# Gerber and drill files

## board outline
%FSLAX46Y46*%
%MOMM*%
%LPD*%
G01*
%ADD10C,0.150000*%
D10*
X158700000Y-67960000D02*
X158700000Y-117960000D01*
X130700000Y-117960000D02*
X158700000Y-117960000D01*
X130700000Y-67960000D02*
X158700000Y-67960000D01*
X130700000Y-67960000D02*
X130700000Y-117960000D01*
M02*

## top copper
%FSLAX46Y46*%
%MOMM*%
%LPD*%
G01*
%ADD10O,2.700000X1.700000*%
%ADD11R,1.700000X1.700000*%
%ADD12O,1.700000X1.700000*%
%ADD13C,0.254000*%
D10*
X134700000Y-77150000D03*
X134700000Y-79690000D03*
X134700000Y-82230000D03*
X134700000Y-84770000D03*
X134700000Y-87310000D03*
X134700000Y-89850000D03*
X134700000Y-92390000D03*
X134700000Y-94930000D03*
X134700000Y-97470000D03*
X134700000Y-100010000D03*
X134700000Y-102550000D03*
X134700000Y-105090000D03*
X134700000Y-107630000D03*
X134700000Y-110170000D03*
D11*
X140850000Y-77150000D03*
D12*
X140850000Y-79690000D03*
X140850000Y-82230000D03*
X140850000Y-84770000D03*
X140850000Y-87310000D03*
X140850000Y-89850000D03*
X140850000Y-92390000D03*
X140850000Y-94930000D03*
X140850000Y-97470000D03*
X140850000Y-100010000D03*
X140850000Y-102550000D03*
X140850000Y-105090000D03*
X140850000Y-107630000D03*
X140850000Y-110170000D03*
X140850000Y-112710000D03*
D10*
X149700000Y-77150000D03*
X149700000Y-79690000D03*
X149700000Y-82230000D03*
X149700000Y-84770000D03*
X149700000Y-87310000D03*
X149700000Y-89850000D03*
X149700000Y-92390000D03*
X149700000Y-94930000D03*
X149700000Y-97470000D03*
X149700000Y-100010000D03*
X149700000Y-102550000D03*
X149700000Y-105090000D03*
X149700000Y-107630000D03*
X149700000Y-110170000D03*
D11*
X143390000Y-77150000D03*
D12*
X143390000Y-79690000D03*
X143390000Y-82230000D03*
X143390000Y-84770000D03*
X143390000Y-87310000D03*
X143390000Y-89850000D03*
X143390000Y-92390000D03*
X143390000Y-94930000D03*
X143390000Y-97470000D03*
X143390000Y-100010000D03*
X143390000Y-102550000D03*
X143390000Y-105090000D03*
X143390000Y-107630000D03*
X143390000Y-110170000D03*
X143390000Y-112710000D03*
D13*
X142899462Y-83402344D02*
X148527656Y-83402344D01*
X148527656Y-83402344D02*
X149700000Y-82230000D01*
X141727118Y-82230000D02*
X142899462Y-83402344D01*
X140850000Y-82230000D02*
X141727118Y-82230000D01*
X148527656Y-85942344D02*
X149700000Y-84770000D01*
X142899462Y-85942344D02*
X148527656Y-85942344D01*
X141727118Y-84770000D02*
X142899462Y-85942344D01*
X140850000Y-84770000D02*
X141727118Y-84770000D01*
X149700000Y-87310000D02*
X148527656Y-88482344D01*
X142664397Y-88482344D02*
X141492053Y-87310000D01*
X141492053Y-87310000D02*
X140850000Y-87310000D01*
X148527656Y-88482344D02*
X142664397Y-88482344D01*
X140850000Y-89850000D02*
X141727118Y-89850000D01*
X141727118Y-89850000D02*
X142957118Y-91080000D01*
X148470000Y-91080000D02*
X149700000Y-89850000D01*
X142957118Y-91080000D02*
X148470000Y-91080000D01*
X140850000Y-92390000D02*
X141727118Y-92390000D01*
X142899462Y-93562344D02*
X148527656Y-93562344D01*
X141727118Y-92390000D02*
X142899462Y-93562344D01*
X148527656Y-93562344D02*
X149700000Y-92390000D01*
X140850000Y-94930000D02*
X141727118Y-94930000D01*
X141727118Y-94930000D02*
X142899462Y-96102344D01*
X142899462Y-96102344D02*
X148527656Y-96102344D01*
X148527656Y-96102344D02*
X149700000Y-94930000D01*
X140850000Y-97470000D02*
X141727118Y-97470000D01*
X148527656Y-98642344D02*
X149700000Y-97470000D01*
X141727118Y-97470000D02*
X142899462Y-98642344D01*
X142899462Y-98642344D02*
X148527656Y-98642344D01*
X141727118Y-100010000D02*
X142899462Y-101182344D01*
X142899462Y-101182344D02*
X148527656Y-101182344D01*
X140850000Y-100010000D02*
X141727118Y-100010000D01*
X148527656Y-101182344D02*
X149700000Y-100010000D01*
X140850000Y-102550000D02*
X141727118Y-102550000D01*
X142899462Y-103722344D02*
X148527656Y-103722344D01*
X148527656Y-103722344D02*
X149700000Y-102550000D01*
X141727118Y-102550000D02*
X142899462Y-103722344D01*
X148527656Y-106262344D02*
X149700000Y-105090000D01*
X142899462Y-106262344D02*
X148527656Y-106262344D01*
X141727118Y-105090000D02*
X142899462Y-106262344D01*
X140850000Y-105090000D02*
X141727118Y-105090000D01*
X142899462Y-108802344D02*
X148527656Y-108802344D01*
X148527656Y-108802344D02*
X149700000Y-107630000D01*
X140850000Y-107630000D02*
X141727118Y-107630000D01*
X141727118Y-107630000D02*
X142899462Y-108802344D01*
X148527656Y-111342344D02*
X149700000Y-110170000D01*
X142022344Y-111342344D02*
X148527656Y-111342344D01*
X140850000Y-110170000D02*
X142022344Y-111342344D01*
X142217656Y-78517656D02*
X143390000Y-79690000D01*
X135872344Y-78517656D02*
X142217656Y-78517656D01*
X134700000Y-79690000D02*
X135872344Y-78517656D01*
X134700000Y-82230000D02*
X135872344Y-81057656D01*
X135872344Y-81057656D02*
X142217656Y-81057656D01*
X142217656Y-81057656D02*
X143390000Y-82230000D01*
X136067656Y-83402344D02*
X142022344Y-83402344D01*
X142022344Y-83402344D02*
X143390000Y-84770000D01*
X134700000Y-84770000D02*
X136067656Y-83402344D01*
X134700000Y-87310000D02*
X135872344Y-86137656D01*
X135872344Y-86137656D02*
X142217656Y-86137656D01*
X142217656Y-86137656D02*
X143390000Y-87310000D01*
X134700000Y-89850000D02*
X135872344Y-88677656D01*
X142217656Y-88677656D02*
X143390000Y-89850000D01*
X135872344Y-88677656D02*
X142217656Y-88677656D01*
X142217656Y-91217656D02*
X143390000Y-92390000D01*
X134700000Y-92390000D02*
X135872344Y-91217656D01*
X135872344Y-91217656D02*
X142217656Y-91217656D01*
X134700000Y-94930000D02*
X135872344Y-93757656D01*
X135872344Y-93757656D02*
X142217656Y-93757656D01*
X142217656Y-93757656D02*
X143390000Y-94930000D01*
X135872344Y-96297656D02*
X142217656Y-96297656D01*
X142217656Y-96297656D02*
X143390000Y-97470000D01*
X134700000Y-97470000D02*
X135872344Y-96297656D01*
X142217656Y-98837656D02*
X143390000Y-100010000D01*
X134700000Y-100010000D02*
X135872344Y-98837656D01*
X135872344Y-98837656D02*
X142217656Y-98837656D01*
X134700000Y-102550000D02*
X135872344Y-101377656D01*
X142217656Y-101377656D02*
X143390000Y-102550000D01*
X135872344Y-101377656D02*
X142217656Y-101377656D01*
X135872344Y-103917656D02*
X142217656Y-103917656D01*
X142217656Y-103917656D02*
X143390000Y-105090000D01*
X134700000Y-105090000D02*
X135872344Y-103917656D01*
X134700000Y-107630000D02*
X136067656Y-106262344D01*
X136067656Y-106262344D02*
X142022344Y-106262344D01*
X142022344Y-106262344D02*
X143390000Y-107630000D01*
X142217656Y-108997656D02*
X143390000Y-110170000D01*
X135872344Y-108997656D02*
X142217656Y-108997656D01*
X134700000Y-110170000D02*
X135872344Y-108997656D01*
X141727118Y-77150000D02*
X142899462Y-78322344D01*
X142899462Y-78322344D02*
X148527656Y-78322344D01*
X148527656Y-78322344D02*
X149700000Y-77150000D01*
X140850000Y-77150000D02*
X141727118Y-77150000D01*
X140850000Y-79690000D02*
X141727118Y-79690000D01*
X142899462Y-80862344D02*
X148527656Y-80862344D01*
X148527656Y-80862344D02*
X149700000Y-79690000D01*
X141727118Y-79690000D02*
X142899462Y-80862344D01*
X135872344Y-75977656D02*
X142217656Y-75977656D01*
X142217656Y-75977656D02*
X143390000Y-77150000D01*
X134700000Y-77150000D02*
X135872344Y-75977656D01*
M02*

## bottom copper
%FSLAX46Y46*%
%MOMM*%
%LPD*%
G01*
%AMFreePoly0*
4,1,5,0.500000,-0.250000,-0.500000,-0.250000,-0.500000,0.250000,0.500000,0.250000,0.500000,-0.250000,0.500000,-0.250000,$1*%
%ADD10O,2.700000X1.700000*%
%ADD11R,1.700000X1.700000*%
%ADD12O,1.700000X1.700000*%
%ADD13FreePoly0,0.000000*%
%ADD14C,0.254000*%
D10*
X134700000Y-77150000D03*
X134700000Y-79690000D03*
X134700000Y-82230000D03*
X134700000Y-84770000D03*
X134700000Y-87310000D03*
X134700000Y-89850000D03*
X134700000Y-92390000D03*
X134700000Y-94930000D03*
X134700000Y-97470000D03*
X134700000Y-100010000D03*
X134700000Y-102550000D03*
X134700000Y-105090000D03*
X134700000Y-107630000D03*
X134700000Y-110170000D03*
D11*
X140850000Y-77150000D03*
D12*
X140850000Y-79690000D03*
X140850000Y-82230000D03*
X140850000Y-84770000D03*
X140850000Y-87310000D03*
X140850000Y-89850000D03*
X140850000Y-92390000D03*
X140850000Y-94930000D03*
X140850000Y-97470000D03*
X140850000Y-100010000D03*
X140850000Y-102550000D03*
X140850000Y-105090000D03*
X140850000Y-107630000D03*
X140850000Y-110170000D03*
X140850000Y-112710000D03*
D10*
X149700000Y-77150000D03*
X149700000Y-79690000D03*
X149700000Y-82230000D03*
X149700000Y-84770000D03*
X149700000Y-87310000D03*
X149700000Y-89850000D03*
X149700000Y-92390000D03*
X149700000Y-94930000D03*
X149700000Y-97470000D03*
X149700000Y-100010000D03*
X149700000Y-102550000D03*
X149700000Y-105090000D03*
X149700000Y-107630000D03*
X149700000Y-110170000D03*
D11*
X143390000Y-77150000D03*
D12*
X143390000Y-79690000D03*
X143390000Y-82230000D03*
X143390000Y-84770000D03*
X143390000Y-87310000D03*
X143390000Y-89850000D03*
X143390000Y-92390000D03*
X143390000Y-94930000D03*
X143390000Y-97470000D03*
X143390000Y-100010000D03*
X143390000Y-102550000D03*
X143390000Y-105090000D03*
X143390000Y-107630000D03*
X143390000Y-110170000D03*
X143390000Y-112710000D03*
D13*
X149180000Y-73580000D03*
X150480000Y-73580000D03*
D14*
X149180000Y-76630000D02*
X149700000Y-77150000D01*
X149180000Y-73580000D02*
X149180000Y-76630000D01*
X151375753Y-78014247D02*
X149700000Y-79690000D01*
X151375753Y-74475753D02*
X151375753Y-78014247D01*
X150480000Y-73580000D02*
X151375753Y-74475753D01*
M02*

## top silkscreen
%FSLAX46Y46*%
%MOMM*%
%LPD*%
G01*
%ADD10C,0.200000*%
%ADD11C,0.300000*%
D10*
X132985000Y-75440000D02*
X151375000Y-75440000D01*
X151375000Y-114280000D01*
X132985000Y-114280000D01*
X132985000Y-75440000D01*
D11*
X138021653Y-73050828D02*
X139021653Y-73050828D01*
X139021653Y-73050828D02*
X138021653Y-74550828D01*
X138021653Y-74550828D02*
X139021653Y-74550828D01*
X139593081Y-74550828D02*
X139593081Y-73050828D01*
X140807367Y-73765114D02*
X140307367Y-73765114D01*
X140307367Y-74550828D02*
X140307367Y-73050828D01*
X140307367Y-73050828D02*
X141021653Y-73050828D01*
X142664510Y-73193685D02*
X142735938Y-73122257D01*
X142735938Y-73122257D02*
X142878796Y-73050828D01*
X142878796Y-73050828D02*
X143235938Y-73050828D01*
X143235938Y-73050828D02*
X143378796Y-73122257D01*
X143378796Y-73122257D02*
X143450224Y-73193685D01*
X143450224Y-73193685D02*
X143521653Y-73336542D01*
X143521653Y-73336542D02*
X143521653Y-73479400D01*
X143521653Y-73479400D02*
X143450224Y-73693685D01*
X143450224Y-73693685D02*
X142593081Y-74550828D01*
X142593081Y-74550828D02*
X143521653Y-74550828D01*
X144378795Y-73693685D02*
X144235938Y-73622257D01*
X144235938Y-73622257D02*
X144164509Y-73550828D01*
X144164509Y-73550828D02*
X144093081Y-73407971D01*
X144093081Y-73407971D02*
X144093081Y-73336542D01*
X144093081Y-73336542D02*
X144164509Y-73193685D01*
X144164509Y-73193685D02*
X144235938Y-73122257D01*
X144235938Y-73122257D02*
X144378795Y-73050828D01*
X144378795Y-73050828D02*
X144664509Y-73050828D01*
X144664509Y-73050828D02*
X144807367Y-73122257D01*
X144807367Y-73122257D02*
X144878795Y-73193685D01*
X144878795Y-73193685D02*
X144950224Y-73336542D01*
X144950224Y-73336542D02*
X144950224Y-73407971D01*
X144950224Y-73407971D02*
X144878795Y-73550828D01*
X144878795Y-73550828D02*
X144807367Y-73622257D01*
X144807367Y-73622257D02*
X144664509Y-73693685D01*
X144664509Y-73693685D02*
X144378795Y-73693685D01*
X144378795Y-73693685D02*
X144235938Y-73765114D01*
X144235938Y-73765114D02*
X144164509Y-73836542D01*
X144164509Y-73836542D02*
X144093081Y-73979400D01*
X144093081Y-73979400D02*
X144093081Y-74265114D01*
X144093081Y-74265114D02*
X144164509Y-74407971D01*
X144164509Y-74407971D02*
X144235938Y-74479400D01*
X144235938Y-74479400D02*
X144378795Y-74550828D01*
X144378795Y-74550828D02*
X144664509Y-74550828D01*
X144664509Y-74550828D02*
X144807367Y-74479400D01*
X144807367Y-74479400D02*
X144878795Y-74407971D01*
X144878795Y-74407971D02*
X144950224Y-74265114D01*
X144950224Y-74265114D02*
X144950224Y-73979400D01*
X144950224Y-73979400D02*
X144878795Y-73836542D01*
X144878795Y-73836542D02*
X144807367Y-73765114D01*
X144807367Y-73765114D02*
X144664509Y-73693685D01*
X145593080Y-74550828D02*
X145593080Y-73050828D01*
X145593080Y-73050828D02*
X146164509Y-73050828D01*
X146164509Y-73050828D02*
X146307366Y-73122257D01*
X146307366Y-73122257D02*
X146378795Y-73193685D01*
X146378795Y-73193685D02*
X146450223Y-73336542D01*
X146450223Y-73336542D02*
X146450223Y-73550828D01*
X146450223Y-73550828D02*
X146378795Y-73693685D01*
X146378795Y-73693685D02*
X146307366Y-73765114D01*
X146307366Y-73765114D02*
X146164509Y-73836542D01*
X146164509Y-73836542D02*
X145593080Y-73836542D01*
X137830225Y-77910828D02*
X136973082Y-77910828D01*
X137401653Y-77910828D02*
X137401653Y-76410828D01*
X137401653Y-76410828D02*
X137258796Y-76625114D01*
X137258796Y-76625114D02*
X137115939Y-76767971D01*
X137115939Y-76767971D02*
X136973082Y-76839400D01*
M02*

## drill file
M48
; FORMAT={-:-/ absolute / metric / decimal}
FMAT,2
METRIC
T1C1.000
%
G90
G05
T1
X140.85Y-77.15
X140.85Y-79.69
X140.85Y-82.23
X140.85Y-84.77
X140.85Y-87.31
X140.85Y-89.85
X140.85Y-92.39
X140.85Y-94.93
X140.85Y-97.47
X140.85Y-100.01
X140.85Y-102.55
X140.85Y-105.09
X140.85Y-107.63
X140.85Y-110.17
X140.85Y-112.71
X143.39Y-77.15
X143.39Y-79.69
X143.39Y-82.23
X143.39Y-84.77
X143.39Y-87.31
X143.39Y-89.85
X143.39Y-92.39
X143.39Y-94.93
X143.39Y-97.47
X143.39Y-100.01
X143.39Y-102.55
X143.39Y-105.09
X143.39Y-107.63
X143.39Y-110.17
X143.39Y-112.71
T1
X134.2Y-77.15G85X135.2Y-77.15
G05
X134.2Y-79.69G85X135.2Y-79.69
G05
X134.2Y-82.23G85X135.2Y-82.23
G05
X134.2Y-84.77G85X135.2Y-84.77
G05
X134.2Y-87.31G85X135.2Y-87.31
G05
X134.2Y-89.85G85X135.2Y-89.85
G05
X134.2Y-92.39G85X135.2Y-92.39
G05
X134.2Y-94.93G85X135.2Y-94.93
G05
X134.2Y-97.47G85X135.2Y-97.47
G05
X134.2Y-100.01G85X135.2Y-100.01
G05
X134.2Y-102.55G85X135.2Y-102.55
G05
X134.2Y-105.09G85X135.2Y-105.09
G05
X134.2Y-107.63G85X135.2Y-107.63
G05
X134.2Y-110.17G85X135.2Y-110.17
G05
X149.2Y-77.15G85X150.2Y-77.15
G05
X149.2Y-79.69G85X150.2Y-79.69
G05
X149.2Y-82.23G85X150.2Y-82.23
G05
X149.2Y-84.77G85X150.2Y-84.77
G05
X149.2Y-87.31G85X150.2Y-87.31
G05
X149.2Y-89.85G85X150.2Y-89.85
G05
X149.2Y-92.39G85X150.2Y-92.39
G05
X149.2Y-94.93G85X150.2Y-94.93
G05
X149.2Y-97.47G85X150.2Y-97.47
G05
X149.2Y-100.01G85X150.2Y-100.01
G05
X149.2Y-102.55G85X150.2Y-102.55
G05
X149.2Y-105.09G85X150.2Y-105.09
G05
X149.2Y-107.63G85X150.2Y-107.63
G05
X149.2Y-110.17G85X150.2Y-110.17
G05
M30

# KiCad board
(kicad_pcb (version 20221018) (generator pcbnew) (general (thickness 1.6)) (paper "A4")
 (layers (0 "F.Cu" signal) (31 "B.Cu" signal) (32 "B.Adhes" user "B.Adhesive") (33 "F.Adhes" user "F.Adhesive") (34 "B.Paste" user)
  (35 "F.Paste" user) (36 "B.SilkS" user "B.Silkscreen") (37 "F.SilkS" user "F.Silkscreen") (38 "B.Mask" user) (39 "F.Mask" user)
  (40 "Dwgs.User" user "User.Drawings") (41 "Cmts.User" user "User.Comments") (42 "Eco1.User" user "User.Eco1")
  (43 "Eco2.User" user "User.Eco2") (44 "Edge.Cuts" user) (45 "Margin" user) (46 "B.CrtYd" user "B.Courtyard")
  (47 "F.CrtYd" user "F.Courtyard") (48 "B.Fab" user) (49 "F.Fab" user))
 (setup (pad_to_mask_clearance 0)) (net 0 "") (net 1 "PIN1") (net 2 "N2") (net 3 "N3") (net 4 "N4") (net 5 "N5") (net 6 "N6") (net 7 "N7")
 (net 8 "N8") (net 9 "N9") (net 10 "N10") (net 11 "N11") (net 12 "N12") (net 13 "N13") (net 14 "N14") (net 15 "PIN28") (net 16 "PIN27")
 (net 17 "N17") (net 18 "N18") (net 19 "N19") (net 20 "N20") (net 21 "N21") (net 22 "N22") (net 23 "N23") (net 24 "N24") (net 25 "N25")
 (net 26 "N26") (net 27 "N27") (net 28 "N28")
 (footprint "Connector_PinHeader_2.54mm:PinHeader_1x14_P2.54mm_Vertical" (layer "F.Cu") (at 134.7 77.15)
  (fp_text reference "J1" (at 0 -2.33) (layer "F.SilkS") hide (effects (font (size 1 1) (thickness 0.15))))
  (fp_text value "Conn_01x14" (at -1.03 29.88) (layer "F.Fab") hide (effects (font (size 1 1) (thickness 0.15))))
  (pad "1" thru_hole oval (at 0 0) (size 2.7 1.7) (drill oval 2 1) (layers "*.Cu" "B.Mask") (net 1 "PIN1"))
  (pad "2" thru_hole oval (at 0 2.54) (size 2.7 1.7) (drill oval 2 1) (layers "*.Cu" "B.Mask") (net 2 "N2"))
  (pad "3" thru_hole oval (at 0 5.08) (size 2.7 1.7) (drill oval 2 1) (layers "*.Cu" "B.Mask") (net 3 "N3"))
  (pad "4" thru_hole oval (at 0 7.62) (size 2.7 1.7) (drill oval 2 1) (layers "*.Cu" "B.Mask") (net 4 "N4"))
  (pad "5" thru_hole oval (at 0 10.16) (size 2.7 1.7) (drill oval 2 1) (layers "*.Cu" "B.Mask") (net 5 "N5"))
  (pad "6" thru_hole oval (at 0 12.7) (size 2.7 1.7) (drill oval 2 1) (layers "*.Cu" "B.Mask") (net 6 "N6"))
  (pad "7" thru_hole oval (at 0 15.24) (size 2.7 1.7) (drill oval 2 1) (layers "*.Cu" "B.Mask") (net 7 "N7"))
  (pad "8" thru_hole oval (at 0 17.78) (size 2.7 1.7) (drill oval 2 1) (layers "*.Cu" "B.Mask") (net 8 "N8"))
  (pad "9" thru_hole oval (at 0 20.32) (size 2.7 1.7) (drill oval 2 1) (layers "*.Cu" "B.Mask") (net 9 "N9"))
  (pad "10" thru_hole oval (at 0 22.86) (size 2.7 1.7) (drill oval 2 1) (layers "*.Cu" "B.Mask") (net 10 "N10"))
  (pad "11" thru_hole oval (at 0 25.4) (size 2.7 1.7) (drill oval 2 1) (layers "*.Cu" "B.Mask") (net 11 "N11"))
  (pad "12" thru_hole oval (at 0 27.94) (size 2.7 1.7) (drill oval 2 1) (layers "*.Cu" "B.Mask") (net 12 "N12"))
  (pad "13" thru_hole oval (at 0 30.48) (size 2.7 1.7) (drill oval 2 1) (layers "*.Cu" "B.Mask") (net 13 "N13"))
  (pad "14" thru_hole oval (at 0 33.02) (size 2.7 1.7) (drill oval 2 1) (layers "*.Cu" "B.Mask") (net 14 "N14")))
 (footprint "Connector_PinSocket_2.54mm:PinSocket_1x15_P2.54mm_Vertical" (layer "F.Cu") (at 140.85 77.15)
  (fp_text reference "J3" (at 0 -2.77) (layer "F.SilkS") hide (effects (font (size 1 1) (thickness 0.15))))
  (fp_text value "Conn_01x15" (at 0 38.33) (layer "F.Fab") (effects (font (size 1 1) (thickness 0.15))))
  (pad "1" thru_hole rect (at 0 0) (size 1.7 1.7) (drill 1) (layers "*.Cu" "F.Mask") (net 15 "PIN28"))
  (pad "2" thru_hole oval (at 0 2.54) (size 1.7 1.7) (drill 1) (layers "*.Cu" "F.Mask") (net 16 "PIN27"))
  (pad "3" thru_hole oval (at 0 5.08) (size 1.7 1.7) (drill 1) (layers "*.Cu" "F.Mask") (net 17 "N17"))
  (pad "4" thru_hole oval (at 0 7.62) (size 1.7 1.7) (drill 1) (layers "*.Cu" "F.Mask") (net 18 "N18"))
  (pad "5" thru_hole oval (at 0 10.16) (size 1.7 1.7) (drill 1) (layers "*.Cu" "F.Mask") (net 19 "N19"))
  (pad "6" thru_hole oval (at 0 12.7) (size 1.7 1.7) (drill 1) (layers "*.Cu" "F.Mask") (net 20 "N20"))
  (pad "7" thru_hole oval (at 0 15.24) (size 1.7 1.7) (drill 1) (layers "*.Cu" "F.Mask") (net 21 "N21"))
  (pad "8" thru_hole oval (at 0 17.78) (size 1.7 1.7) (drill 1) (layers "*.Cu" "F.Mask") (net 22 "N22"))
  (pad "9" thru_hole oval (at 0 20.32) (size 1.7 1.7) (drill 1) (layers "*.Cu" "F.Mask") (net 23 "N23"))
  (pad "10" thru_hole oval (at 0 22.86) (size 1.7 1.7) (drill 1) (layers "*.Cu" "F.Mask") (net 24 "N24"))
  (pad "11" thru_hole oval (at 0 25.4) (size 1.7 1.7) (drill 1) (layers "*.Cu" "F.Mask") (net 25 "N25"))
  (pad "12" thru_hole oval (at 0 27.94) (size 1.7 1.7) (drill 1) (layers "*.Cu" "F.Mask") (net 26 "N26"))
  (pad "13" thru_hole oval (at 0 30.48) (size 1.7 1.7) (drill 1) (layers "*.Cu" "F.Mask") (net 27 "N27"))
  (pad "14" thru_hole oval (at 0 33.02) (size 1.7 1.7) (drill 1) (layers "*.Cu" "F.Mask") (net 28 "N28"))
  (pad "15" thru_hole oval (at 0 35.56) (size 1.7 1.7) (drill 1) (layers "*.Cu" "F.Mask")))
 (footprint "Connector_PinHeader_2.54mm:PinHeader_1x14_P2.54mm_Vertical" (layer "F.Cu") (at 149.7 77.15)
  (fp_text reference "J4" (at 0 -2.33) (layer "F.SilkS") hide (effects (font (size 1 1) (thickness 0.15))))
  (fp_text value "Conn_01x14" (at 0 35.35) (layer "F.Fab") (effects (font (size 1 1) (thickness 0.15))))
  (pad "1" thru_hole oval (at 0 0) (size 2.7 1.7) (drill oval 2 1) (layers "*.Cu" "B.Mask") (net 15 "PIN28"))
  (pad "2" thru_hole oval (at 0 2.54) (size 2.7 1.7) (drill oval 2 1) (layers "*.Cu" "B.Mask") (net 16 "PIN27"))
  (pad "3" thru_hole oval (at 0 5.08) (size 2.7 1.7) (drill oval 2 1) (layers "*.Cu" "B.Mask") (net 17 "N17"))
  (pad "4" thru_hole oval (at 0 7.62) (size 2.7 1.7) (drill oval 2 1) (layers "*.Cu" "B.Mask") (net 18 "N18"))
  (pad "5" thru_hole oval (at 0 10.16) (size 2.7 1.7) (drill oval 2 1) (layers "*.Cu" "B.Mask") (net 19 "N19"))
  (pad "6" thru_hole oval (at 0 12.7) (size 2.7 1.7) (drill oval 2 1) (layers "*.Cu" "B.Mask") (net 20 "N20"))
  (pad "7" thru_hole oval (at 0 15.24) (size 2.7 1.7) (drill oval 2 1) (layers "*.Cu" "B.Mask") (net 21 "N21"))
  (pad "8" thru_hole oval (at 0 17.78) (size 2.7 1.7) (drill oval 2 1) (layers "*.Cu" "B.Mask") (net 22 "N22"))
  (pad "9" thru_hole oval (at 0 20.32) (size 2.7 1.7) (drill oval 2 1) (layers "*.Cu" "B.Mask") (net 23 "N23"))
  (pad "10" thru_hole oval (at 0 22.86) (size 2.7 1.7) (drill oval 2 1) (layers "*.Cu" "B.Mask") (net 24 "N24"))
  (pad "11" thru_hole oval (at 0 25.4) (size 2.7 1.7) (drill oval 2 1) (layers "*.Cu" "B.Mask") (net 25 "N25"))
  (pad "12" thru_hole oval (at 0 27.94) (size 2.7 1.7) (drill oval 2 1) (layers "*.Cu" "B.Mask") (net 26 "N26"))
  (pad "13" thru_hole oval (at 0 30.48) (size 2.7 1.7) (drill oval 2 1) (layers "*.Cu" "B.Mask") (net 27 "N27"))
  (pad "14" thru_hole oval (at 0 33.02) (size 2.7 1.7) (drill oval 2 1) (layers "*.Cu" "B.Mask") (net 28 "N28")))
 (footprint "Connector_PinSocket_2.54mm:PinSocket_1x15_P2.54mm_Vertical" (layer "F.Cu") (at 143.39 77.15)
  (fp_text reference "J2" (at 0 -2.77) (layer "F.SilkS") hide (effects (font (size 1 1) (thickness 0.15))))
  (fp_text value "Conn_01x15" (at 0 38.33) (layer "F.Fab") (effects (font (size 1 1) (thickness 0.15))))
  (pad "1" thru_hole rect (at 0 0) (size 1.7 1.7) (drill 1) (layers "*.Cu" "F.Mask") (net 1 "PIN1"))
  (pad "2" thru_hole oval (at 0 2.54) (size 1.7 1.7) (drill 1) (layers "*.Cu" "F.Mask") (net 2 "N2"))
  (pad "3" thru_hole oval (at 0 5.08) (size 1.7 1.7) (drill 1) (layers "*.Cu" "F.Mask") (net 3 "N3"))
  (pad "4" thru_hole oval (at 0 7.62) (size 1.7 1.7) (drill 1) (layers "*.Cu" "F.Mask") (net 4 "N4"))
  (pad "5" thru_hole oval (at 0 10.16) (size 1.7 1.7) (drill 1) (layers "*.Cu" "F.Mask") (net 5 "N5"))
  (pad "6" thru_hole oval (at 0 12.7) (size 1.7 1.7) (drill 1) (layers "*.Cu" "F.Mask") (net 6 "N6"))
  (pad "7" thru_hole oval (at 0 15.24) (size 1.7 1.7) (drill 1) (layers "*.Cu" "F.Mask") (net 7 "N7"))
  (pad "8" thru_hole oval (at 0 17.78) (size 1.7 1.7) (drill 1) (layers "*.Cu" "F.Mask") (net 8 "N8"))
  (pad "9" thru_hole oval (at 0 20.32) (size 1.7 1.7) (drill 1) (layers "*.Cu" "F.Mask") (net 9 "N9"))
  (pad "10" thru_hole oval (at 0 22.86) (size 1.7 1.7) (drill 1) (layers "*.Cu" "F.Mask") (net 10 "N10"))
  (pad "11" thru_hole oval (at 0 25.4) (size 1.7 1.7) (drill 1) (layers "*.Cu" "F.Mask") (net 11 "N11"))
  (pad "12" thru_hole oval (at 0 27.94) (size 1.7 1.7) (drill 1) (layers "*.Cu" "F.Mask") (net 12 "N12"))
  (pad "13" thru_hole oval (at 0 30.48) (size 1.7 1.7) (drill 1) (layers "*.Cu" "F.Mask") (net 13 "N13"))
  (pad "14" thru_hole oval (at 0 33.02) (size 1.7 1.7) (drill 1) (layers "*.Cu" "F.Mask") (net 14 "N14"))
  (pad "15" thru_hole oval (at 0 35.56) (size 1.7 1.7) (drill 1) (layers "*.Cu" "F.Mask")))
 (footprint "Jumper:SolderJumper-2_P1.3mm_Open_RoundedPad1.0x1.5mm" (layer "B.Cu") (at 149.83 73.58)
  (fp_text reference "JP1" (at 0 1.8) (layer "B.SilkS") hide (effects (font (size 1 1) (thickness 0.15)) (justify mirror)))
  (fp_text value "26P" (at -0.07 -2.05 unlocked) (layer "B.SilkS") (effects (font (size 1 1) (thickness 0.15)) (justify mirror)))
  (pad "1" smd custom (at -0.65 0) (size 1 0.5) (layers "B.Cu" "B.Mask") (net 15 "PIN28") (zone_connect 2)
   (options (clearance outline) (anchor rect)) (primitives))
  (pad "2" smd custom (at 0.65 0) (size 1 0.5) (layers "B.Cu" "B.Mask") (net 16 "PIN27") (zone_connect 2)
   (options (clearance outline) (anchor rect)) (primitives)))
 (gr_rect (start 132.985 75.44) (end 151.375 114.28) (stroke (width 0.2) (type default)) (fill none) (layer "F.SilkS"))
 (gr_line (start 158.7 67.96) (end 158.7 117.96) (stroke (width 0.15) (type solid)) (layer "Edge.Cuts"))
 (gr_line (start 130.7 117.96) (end 158.7 117.96) (stroke (width 0.15) (type solid)) (layer "Edge.Cuts"))
 (gr_line (start 130.7 67.96) (end 158.7 67.96) (stroke (width 0.15) (type solid)) (layer "Edge.Cuts"))
 (gr_line (start 130.7 67.96) (end 130.7 117.96) (stroke (width 0.15) (type solid)) (layer "Edge.Cuts"))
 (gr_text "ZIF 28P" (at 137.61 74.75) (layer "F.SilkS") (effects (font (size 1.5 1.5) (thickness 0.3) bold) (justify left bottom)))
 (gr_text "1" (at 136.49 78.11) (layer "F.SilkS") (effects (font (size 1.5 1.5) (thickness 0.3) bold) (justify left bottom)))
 (segment (start 142.899462 83.402344) (end 148.527656 83.402344) (width 0.254) (layer "F.Cu") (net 17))
 (segment (start 148.527656 83.402344) (end 149.7 82.23) (width 0.254) (layer "F.Cu") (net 17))
 (segment (start 141.727118 82.23) (end 142.899462 83.402344) (width 0.254) (layer "F.Cu") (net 17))
 (segment (start 140.85 82.23) (end 141.727118 82.23) (width 0.254) (layer "F.Cu") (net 17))
 (segment (start 148.527656 85.942344) (end 149.7 84.77) (width 0.254) (layer "F.Cu") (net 18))
 (segment (start 142.899462 85.942344) (end 148.527656 85.942344) (width 0.254) (layer "F.Cu") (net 18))
 (segment (start 141.727118 84.77) (end 142.899462 85.942344) (width 0.254) (layer "F.Cu") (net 18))
 (segment (start 140.85 84.77) (end 141.727118 84.77) (width 0.254) (layer "F.Cu") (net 18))
 (segment (start 149.7 87.31) (end 148.527656 88.482344) (width 0.254) (layer "F.Cu") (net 19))
 (segment (start 142.664397 88.482344) (end 141.492053 87.31) (width 0.254) (layer "F.Cu") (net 19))
 (segment (start 141.492053 87.31) (end 140.85 87.31) (width 0.254) (layer "F.Cu") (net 19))
 (segment (start 148.527656 88.482344) (end 142.664397 88.482344) (width 0.254) (layer "F.Cu") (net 19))
 (segment (start 140.85 89.85) (end 141.727118 89.85) (width 0.254) (layer "F.Cu") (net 20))
 (segment (start 141.727118 89.85) (end 142.957118 91.08) (width 0.254) (layer "F.Cu") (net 20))
 (segment (start 148.47 91.08) (end 149.7 89.85) (width 0.254) (layer "F.Cu") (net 20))
 (segment (start 142.957118 91.08) (end 148.47 91.08) (width 0.254) (layer "F.Cu") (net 20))
 (segment (start 140.85 92.39) (end 141.727118 92.39) (width 0.254) (layer "F.Cu") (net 21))
 (segment (start 142.899462 93.562344) (end 148.527656 93.562344) (width 0.254) (layer "F.Cu") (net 21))
 (segment (start 141.727118 92.39) (end 142.899462 93.562344) (width 0.254) (layer "F.Cu") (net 21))
 (segment (start 148.527656 93.562344) (end 149.7 92.39) (width 0.254) (layer "F.Cu") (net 21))
 (segment (start 140.85 94.93) (end 141.727118 94.93) (width 0.254) (layer "F.Cu") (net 22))
 (segment (start 141.727118 94.93) (end 142.899462 96.102344) (width 0.254) (layer "F.Cu") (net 22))
 (segment (start 142.899462 96.102344) (end 148.527656 96.102344) (width 0.254) (layer "F.Cu") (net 22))
 (segment (start 148.527656 96.102344) (end 149.7 94.93) (width 0.254) (layer "F.Cu") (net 22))
 (segment (start 140.85 97.47) (end 141.727118 97.47) (width 0.254) (layer "F.Cu") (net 23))
 (segment (start 148.527656 98.642344) (end 149.7 97.47) (width 0.254) (layer "F.Cu") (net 23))
 (segment (start 141.727118 97.47) (end 142.899462 98.642344) (width 0.254) (layer "F.Cu") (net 23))
 (segment (start 142.899462 98.642344) (end 148.527656 98.642344) (width 0.254) (layer "F.Cu") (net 23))
 (segment (start 141.727118 100.01) (end 142.899462 101.182344) (width 0.254) (layer "F.Cu") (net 24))
 (segment (start 142.899462 101.182344) (end 148.527656 101.182344) (width 0.254) (layer "F.Cu") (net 24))
 (segment (start 140.85 100.01) (end 141.727118 100.01) (width 0.254) (layer "F.Cu") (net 24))
 (segment (start 148.527656 101.182344) (end 149.7 100.01) (width 0.254) (layer "F.Cu") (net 24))
 (segment (start 140.85 102.55) (end 141.727118 102.55) (width 0.254) (layer "F.Cu") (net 25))
 (segment (start 142.899462 103.722344) (end 148.527656 103.722344) (width 0.254) (layer "F.Cu") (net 25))
 (segment (start 148.527656 103.722344) (end 149.7 102.55) (width 0.254) (layer "F.Cu") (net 25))
 (segment (start 141.727118 102.55) (end 142.899462 103.722344) (width 0.254) (layer "F.Cu") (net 25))
 (segment (start 148.527656 106.262344) (end 149.7 105.09) (width 0.254) (layer "F.Cu") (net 26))
 (segment (start 142.899462 106.262344) (end 148.527656 106.262344) (width 0.254) (layer "F.Cu") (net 26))
 (segment (start 141.727118 105.09) (end 142.899462 106.262344) (width 0.254) (layer "F.Cu") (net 26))
 (segment (start 140.85 105.09) (end 141.727118 105.09) (width 0.254) (layer "F.Cu") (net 26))
 (segment (start 142.899462 108.802344) (end 148.527656 108.802344) (width 0.254) (layer "F.Cu") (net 27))
 (segment (start 148.527656 108.802344) (end 149.7 107.63) (width 0.254) (layer "F.Cu") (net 27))
 (segment (start 140.85 107.63) (end 141.727118 107.63) (width 0.254) (layer "F.Cu") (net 27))
 (segment (start 141.727118 107.63) (end 142.899462 108.802344) (width 0.254) (layer "F.Cu") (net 27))
 (segment (start 148.527656 111.342344) (end 149.7 110.17) (width 0.254) (layer "F.Cu") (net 28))
 (segment (start 142.022344 111.342344) (end 148.527656 111.342344) (width 0.254) (layer "F.Cu") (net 28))
 (segment (start 140.85 110.17) (end 142.022344 111.342344) (width 0.254) (layer "F.Cu") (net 28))
 (segment (start 142.217656 78.517656) (end 143.39 79.69) (width 0.254) (layer "F.Cu") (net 2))
 (segment (start 135.872344 78.517656) (end 142.217656 78.517656) (width 0.254) (layer "F.Cu") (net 2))
 (segment (start 134.7 79.69) (end 135.872344 78.517656) (width 0.254) (layer "F.Cu") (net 2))
 (segment (start 134.7 82.23) (end 135.872344 81.057656) (width 0.254) (layer "F.Cu") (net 3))
 (segment (start 135.872344 81.057656) (end 142.217656 81.057656) (width 0.254) (layer "F.Cu") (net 3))
 (segment (start 142.217656 81.057656) (end 143.39 82.23) (width 0.254) (layer "F.Cu") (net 3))
 (segment (start 136.067656 83.402344) (end 142.022344 83.402344) (width 0.254) (layer "F.Cu") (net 4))
 (segment (start 142.022344 83.402344) (end 143.39 84.77) (width 0.254) (layer "F.Cu") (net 4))
 (segment (start 134.7 84.77) (end 136.067656 83.402344) (width 0.254) (layer "F.Cu") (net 4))
 (segment (start 134.7 87.31) (end 135.872344 86.137656) (width 0.254) (layer "F.Cu") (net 5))
 (segment (start 135.872344 86.137656) (end 142.217656 86.137656) (width 0.254) (layer "F.Cu") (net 5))
 (segment (start 142.217656 86.137656) (end 143.39 87.31) (width 0.254) (layer "F.Cu") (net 5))
 (segment (start 134.7 89.85) (end 135.872344 88.677656) (width 0.254) (layer "F.Cu") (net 6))
 (segment (start 142.217656 88.677656) (end 143.39 89.85) (width 0.254) (layer "F.Cu") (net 6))
 (segment (start 135.872344 88.677656) (end 142.217656 88.677656) (width 0.254) (layer "F.Cu") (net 6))
 (segment (start 142.217656 91.217656) (end 143.39 92.39) (width 0.254) (layer "F.Cu") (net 7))
 (segment (start 134.7 92.39) (end 135.872344 91.217656) (width 0.254) (layer "F.Cu") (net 7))
 (segment (start 135.872344 91.217656) (end 142.217656 91.217656) (width 0.254) (layer "F.Cu") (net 7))
 (segment (start 134.7 94.93) (end 135.872344 93.757656) (width 0.254) (layer "F.Cu") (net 8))
 (segment (start 135.872344 93.757656) (end 142.217656 93.757656) (width 0.254) (layer "F.Cu") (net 8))
 (segment (start 142.217656 93.757656) (end 143.39 94.93) (width 0.254) (layer "F.Cu") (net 8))
 (segment (start 135.872344 96.297656) (end 142.217656 96.297656) (width 0.254) (layer "F.Cu") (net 9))
 (segment (start 142.217656 96.297656) (end 143.39 97.47) (width 0.254) (layer "F.Cu") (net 9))
 (segment (start 134.7 97.47) (end 135.872344 96.297656) (width 0.254) (layer "F.Cu") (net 9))
 (segment (start 142.217656 98.837656) (end 143.39 100.01) (width 0.254) (layer "F.Cu") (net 10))
 (segment (start 134.7 100.01) (end 135.872344 98.837656) (width 0.254) (layer "F.Cu") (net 10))
 (segment (start 135.872344 98.837656) (end 142.217656 98.837656) (width 0.254) (layer "F.Cu") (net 10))
 (segment (start 134.7 102.55) (end 135.872344 101.377656) (width 0.254) (layer "F.Cu") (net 11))
 (segment (start 142.217656 101.377656) (end 143.39 102.55) (width 0.254) (layer "F.Cu") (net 11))
 (segment (start 135.872344 101.377656) (end 142.217656 101.377656) (width 0.254) (layer "F.Cu") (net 11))
 (segment (start 135.872344 103.917656) (end 142.217656 103.917656) (width 0.254) (layer "F.Cu") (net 12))
 (segment (start 142.217656 103.917656) (end 143.39 105.09) (width 0.254) (layer "F.Cu") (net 12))
 (segment (start 134.7 105.09) (end 135.872344 103.917656) (width 0.254) (layer "F.Cu") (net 12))
 (segment (start 134.7 107.63) (end 136.067656 106.262344) (width 0.254) (layer "F.Cu") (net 13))
 (segment (start 136.067656 106.262344) (end 142.022344 106.262344) (width 0.254) (layer "F.Cu") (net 13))
 (segment (start 142.022344 106.262344) (end 143.39 107.63) (width 0.254) (layer "F.Cu") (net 13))
 (segment (start 142.217656 108.997656) (end 143.39 110.17) (width 0.254) (layer "F.Cu") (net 14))
 (segment (start 135.872344 108.997656) (end 142.217656 108.997656) (width 0.254) (layer "F.Cu") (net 14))
 (segment (start 134.7 110.17) (end 135.872344 108.997656) (width 0.254) (layer "F.Cu") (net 14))
 (segment (start 141.727118 77.15) (end 142.899462 78.322344) (width 0.254) (layer "F.Cu") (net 15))
 (segment (start 142.899462 78.322344) (end 148.527656 78.322344) (width 0.254) (layer "F.Cu") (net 15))
 (segment (start 148.527656 78.322344) (end 149.7 77.15) (width 0.254) (layer "F.Cu") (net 15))
 (segment (start 140.85 77.15) (end 141.727118 77.15) (width 0.254) (layer "F.Cu") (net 15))
 (segment (start 149.18 76.63) (end 149.7 77.15) (width 0.254) (layer "B.Cu") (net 15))
 (segment (start 149.18 73.58) (end 149.18 76.63) (width 0.254) (layer "B.Cu") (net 15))
 (segment (start 140.85 79.69) (end 141.727118 79.69) (width 0.254) (layer "F.Cu") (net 16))
 (segment (start 142.899462 80.862344) (end 148.527656 80.862344) (width 0.254) (layer "F.Cu") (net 16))
 (segment (start 148.527656 80.862344) (end 149.7 79.69) (width 0.254) (layer "F.Cu") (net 16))
 (segment (start 141.727118 79.69) (end 142.899462 80.862344) (width 0.254) (layer "F.Cu") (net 16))
 (segment (start 151.375753 78.014247) (end 149.7 79.69) (width 0.254) (layer "B.Cu") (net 16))
 (segment (start 151.375753 74.475753) (end 151.375753 78.014247) (width 0.254) (layer "B.Cu") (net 16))
 (segment (start 150.48 73.58) (end 151.375753 74.475753) (width 0.254) (layer "B.Cu") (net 16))
 (segment (start 135.872344 75.977656) (end 142.217656 75.977656) (width 0.254) (layer "F.Cu") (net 1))
 (segment (start 142.217656 75.977656) (end 143.39 77.15) (width 0.254) (layer "F.Cu") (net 1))
 (segment (start 134.7 77.15) (end 135.872344 75.977656) (width 0.254) (layer "F.Cu") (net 1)))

